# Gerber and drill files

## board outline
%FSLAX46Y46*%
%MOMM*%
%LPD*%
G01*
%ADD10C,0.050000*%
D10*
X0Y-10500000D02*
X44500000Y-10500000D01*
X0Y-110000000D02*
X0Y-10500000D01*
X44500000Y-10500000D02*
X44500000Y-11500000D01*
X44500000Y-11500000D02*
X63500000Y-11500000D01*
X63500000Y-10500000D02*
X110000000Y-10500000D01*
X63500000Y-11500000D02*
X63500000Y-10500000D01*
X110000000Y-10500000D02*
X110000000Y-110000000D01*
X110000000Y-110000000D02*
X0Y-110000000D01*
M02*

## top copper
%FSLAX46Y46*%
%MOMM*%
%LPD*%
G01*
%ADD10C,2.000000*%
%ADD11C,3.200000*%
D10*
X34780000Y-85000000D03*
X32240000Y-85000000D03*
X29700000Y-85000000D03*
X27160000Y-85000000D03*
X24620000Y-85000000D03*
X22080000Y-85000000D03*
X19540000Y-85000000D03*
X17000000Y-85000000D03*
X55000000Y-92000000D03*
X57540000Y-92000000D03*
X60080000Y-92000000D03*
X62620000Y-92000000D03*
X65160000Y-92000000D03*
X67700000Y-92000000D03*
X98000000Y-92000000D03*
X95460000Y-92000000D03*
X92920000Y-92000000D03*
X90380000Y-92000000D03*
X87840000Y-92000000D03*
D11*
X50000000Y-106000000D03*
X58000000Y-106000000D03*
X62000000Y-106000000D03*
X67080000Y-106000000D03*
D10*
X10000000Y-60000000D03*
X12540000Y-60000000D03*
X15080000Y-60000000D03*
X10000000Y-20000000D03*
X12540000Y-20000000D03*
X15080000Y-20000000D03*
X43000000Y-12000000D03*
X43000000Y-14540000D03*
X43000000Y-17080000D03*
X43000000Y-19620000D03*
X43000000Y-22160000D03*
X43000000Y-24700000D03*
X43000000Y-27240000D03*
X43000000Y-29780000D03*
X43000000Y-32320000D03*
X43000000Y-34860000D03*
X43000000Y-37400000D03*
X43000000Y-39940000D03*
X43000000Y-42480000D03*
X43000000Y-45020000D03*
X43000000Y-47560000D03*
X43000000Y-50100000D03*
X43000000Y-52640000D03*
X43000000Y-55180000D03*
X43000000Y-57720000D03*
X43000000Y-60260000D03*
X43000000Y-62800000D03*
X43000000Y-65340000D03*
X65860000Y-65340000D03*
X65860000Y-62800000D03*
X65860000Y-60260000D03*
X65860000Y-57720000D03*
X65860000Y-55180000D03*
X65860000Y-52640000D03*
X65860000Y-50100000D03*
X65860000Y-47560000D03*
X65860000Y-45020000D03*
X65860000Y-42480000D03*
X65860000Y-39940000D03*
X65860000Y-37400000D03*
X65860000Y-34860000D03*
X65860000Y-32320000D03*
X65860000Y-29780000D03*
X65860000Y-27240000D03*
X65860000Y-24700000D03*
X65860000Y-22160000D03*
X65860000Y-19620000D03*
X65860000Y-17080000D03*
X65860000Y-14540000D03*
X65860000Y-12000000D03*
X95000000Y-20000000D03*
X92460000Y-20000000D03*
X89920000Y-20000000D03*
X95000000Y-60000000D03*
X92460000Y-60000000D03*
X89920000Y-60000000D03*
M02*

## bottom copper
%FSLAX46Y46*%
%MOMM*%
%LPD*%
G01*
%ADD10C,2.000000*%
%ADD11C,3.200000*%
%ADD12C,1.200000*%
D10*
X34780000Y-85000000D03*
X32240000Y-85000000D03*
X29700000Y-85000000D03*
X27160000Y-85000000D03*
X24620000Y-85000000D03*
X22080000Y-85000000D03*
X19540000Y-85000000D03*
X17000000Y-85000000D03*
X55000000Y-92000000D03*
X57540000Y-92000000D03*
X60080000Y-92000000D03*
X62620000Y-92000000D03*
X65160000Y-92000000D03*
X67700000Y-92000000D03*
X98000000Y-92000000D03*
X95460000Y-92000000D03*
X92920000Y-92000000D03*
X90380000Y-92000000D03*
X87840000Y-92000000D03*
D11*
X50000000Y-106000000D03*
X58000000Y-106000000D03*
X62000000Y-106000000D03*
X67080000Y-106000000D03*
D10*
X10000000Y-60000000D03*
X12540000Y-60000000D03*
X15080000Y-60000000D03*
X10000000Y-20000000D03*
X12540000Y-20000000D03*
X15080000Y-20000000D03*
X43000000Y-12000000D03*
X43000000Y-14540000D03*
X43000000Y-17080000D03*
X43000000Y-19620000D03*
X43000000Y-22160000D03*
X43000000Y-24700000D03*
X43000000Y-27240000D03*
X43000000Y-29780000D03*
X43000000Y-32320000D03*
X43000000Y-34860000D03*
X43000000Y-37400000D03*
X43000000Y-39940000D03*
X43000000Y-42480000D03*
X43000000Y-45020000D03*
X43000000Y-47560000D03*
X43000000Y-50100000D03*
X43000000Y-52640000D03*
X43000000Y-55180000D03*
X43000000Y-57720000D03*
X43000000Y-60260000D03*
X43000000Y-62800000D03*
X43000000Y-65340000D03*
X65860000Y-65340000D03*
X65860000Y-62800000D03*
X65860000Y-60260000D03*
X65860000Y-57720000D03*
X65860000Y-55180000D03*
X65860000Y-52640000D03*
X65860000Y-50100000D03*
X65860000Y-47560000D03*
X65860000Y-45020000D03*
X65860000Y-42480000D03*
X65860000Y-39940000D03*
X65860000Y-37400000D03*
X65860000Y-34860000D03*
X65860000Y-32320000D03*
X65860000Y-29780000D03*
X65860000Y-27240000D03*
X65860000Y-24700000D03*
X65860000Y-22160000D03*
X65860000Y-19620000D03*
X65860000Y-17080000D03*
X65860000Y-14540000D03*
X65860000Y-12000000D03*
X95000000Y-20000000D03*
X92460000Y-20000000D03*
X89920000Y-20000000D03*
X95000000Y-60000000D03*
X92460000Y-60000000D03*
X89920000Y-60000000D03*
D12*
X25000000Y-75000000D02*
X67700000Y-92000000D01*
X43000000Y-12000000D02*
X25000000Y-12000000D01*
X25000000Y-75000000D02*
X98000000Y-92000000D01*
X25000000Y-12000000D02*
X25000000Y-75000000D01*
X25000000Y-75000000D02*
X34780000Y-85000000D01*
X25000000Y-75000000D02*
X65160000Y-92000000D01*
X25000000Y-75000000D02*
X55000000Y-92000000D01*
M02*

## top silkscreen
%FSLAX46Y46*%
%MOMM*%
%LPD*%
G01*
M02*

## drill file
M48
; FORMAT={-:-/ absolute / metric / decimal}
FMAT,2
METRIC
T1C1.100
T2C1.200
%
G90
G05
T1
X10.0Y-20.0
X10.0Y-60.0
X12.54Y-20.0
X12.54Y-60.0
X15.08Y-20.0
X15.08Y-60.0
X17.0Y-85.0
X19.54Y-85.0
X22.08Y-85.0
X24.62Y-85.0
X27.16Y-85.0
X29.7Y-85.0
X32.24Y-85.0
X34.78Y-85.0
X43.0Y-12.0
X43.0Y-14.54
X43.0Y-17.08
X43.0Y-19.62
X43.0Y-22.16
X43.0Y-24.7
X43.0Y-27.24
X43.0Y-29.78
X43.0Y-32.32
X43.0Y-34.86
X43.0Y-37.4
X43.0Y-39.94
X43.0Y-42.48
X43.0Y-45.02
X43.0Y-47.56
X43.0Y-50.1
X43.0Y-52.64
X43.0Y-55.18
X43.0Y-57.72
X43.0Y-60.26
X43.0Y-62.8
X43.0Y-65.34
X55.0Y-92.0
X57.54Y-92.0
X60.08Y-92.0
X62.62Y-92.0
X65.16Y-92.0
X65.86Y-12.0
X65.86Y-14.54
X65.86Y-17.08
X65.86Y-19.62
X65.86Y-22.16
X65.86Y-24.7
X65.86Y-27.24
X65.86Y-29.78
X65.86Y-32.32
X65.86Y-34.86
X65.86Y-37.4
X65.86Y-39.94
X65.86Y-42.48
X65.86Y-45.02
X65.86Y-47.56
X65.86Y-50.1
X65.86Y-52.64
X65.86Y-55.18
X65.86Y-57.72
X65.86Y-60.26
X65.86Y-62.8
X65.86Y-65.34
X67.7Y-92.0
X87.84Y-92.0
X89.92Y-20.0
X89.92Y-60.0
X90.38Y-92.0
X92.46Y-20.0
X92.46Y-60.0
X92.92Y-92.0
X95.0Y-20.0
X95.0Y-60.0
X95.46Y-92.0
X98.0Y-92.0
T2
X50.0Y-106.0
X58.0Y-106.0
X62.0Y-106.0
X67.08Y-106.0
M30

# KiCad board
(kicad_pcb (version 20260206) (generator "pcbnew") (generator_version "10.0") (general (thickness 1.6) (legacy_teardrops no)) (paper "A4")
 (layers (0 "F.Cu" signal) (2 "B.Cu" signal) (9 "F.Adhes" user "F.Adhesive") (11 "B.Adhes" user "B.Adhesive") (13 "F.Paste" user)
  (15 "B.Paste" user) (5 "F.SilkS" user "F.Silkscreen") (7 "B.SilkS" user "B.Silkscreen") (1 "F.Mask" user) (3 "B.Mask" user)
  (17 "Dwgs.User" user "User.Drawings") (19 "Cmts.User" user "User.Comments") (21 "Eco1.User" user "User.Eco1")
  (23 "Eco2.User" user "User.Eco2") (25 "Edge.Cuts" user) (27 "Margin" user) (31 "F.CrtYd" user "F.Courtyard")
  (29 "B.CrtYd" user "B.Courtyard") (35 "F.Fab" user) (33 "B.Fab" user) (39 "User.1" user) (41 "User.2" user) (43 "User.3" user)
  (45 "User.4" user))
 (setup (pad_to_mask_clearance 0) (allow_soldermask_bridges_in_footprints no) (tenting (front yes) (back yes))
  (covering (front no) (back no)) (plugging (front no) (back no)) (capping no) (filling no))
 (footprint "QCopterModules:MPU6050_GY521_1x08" (layer "F.Cu") (at 34.78 85 -90)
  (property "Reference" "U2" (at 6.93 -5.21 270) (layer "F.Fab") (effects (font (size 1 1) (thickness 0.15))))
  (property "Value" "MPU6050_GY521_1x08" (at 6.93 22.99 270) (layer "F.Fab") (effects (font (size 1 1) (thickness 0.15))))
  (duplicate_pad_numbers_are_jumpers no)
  (pad "1" thru_hole circle (at 0 0 270) (size 2 2) (drill 1.1) (layers "*.Cu" "*.Mask") (remove_unused_layers no) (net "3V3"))
  (pad "2" thru_hole circle (at 0 2.54 270) (size 2 2) (drill 1.1) (layers "*.Cu" "*.Mask") (remove_unused_layers no) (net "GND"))
  (pad "3" thru_hole circle (at 0 5.08 270) (size 2 2) (drill 1.1) (layers "*.Cu" "*.Mask") (remove_unused_layers no) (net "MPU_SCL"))
  (pad "4" thru_hole circle (at 0 7.62 270) (size 2 2) (drill 1.1) (layers "*.Cu" "*.Mask") (remove_unused_layers no) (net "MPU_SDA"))
  (pad "5" thru_hole circle (at 0 10.16 270) (size 2 2) (drill 1.1) (layers "*.Cu" "*.Mask") (remove_unused_layers no)
   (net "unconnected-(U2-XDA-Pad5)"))
  (pad "6" thru_hole circle (at 0 12.7 270) (size 2 2) (drill 1.1) (layers "*.Cu" "*.Mask") (remove_unused_layers no)
   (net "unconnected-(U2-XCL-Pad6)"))
  (pad "7" thru_hole circle (at 0 15.24 270) (size 2 2) (drill 1.1) (layers "*.Cu" "*.Mask") (remove_unused_layers no) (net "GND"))
  (pad "8" thru_hole circle (at 0 17.78 270) (size 2 2) (drill 1.1) (layers "*.Cu" "*.Mask") (remove_unused_layers no) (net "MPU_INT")))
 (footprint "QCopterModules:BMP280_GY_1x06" (layer "F.Cu") (at 55 92 90)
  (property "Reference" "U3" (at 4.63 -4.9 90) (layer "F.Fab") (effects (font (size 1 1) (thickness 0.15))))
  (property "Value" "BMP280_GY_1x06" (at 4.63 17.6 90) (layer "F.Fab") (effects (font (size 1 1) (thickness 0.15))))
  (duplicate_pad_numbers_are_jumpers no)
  (pad "1" thru_hole circle (at 0 0 90) (size 2 2) (drill 1.1) (layers "*.Cu" "*.Mask") (remove_unused_layers no) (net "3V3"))
  (pad "2" thru_hole circle (at 0 2.54 90) (size 2 2) (drill 1.1) (layers "*.Cu" "*.Mask") (remove_unused_layers no) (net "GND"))
  (pad "3" thru_hole circle (at 0 5.08 90) (size 2 2) (drill 1.1) (layers "*.Cu" "*.Mask") (remove_unused_layers no) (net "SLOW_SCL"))
  (pad "4" thru_hole circle (at 0 7.62 90) (size 2 2) (drill 1.1) (layers "*.Cu" "*.Mask") (remove_unused_layers no) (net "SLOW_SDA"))
  (pad "5" thru_hole circle (at 0 10.16 90) (size 2 2) (drill 1.1) (layers "*.Cu" "*.Mask") (remove_unused_layers no) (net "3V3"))
  (pad "6" thru_hole circle (at 0 12.7 90) (size 2 2) (drill 1.1) (layers "*.Cu" "*.Mask") (remove_unused_layers no) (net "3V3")))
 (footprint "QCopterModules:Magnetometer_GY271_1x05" (layer "F.Cu") (at 98 92 -90)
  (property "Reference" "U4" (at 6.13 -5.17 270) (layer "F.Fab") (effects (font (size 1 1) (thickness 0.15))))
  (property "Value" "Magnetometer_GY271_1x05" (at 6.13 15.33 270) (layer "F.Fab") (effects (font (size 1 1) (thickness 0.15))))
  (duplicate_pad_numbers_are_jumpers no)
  (pad "1" thru_hole circle (at 0 0 270) (size 2 2) (drill 1.1) (layers "*.Cu" "*.Mask") (remove_unused_layers no) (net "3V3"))
  (pad "2" thru_hole circle (at 0 2.54 270) (size 2 2) (drill 1.1) (layers "*.Cu" "*.Mask") (remove_unused_layers no) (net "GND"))
  (pad "3" thru_hole circle (at 0 5.08 270) (size 2 2) (drill 1.1) (layers "*.Cu" "*.Mask") (remove_unused_layers no) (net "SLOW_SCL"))
  (pad "4" thru_hole circle (at 0 7.62 270) (size 2 2) (drill 1.1) (layers "*.Cu" "*.Mask") (remove_unused_layers no) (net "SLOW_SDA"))
  (pad "5" thru_hole circle (at 0 10.16 270) (size 2 2) (drill 1.1) (layers "*.Cu" "*.Mask") (remove_unused_layers no) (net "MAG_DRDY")))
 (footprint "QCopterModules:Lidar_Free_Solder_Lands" (layer "F.Cu") (at 50 106)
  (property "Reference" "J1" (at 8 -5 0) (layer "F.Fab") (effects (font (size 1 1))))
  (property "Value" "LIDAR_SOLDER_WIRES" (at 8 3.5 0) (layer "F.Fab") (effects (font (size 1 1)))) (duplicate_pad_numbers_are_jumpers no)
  (pad "1" thru_hole circle (at 0 0) (size 3.2 3.2) (drill 1.2) (layers "*.Cu" "*.Mask") (remove_unused_layers no) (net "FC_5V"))
  (pad "2" thru_hole circle (at 8 0) (size 3.2 3.2) (drill 1.2) (layers "*.Cu" "*.Mask") (remove_unused_layers no) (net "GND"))
  (pad "3" thru_hole circle (at 12 0) (size 3.2 3.2) (drill 1.2) (layers "*.Cu" "*.Mask") (remove_unused_layers no) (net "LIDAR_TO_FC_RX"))
  (pad "4" thru_hole circle (at 17.08 0) (size 3.2 3.2) (drill 1.2) (layers "*.Cu" "*.Mask") (remove_unused_layers no)
   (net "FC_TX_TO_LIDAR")))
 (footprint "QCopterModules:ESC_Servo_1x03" (layer "F.Cu") (at 10 60 90)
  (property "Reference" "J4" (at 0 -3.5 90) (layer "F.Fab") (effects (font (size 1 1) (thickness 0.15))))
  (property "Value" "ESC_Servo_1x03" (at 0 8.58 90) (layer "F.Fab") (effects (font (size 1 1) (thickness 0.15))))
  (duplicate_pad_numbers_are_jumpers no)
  (pad "1" thru_hole circle (at 0 0 90) (size 2 2) (drill 1.1) (layers "*.Cu" "*.Mask") (remove_unused_layers no) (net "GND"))
  (pad "2" thru_hole circle (at 0 2.54 90) (size 2 2) (drill 1.1) (layers "*.Cu" "*.Mask") (remove_unused_layers no) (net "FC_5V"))
  (pad "3" thru_hole circle (at 0 5.08 90) (size 2 2) (drill 1.1) (layers "*.Cu" "*.Mask") (remove_unused_layers no) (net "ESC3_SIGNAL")))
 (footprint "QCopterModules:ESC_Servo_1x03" (layer "F.Cu") (at 10 20 90)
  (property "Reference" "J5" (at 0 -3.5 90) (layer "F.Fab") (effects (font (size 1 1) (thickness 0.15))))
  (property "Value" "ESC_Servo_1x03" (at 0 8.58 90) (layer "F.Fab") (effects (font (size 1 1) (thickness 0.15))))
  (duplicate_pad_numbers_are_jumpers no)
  (pad "1" thru_hole circle (at 0 0 90) (size 2 2) (drill 1.1) (layers "*.Cu" "*.Mask") (remove_unused_layers no) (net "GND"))
  (pad "2" thru_hole circle (at 0 2.54 90) (size 2 2) (drill 1.1) (layers "*.Cu" "*.Mask") (remove_unused_layers no)
   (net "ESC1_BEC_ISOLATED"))
  (pad "3" thru_hole circle (at 0 5.08 90) (size 2 2) (drill 1.1) (layers "*.Cu" "*.Mask") (remove_unused_layers no) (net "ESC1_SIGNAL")))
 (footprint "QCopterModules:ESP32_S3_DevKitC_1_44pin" (layer "F.Cu") (at 43 12)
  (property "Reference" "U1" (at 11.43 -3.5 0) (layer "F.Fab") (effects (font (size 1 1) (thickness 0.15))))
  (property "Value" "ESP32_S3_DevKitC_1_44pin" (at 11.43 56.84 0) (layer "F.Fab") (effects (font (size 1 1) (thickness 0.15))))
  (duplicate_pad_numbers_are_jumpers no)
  (pad "1" thru_hole circle (at 0 0) (size 2 2) (drill 1.1) (layers "*.Cu" "*.Mask") (remove_unused_layers no) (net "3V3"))
  (pad "2" thru_hole circle (at 0 2.54) (size 2 2) (drill 1.1) (layers "*.Cu" "*.Mask") (remove_unused_layers no))
  (pad "3" thru_hole circle (at 0 5.08) (size 2 2) (drill 1.1) (layers "*.Cu" "*.Mask") (remove_unused_layers no)
   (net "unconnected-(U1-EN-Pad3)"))
  (pad "4" thru_hole circle (at 0 7.62) (size 2 2) (drill 1.1) (layers "*.Cu" "*.Mask") (remove_unused_layers no) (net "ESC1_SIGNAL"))
  (pad "5" thru_hole circle (at 0 10.16) (size 2 2) (drill 1.1) (layers "*.Cu" "*.Mask") (remove_unused_layers no)
   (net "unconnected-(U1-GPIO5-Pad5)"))
  (pad "6" thru_hole circle (at 0 12.7) (size 2 2) (drill 1.1) (layers "*.Cu" "*.Mask") (remove_unused_layers no)
   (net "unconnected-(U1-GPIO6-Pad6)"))
  (pad "7" thru_hole circle (at 0 15.24) (size 2 2) (drill 1.1) (layers "*.Cu" "*.Mask") (remove_unused_layers no)
   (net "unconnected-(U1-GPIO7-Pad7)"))
  (pad "8" thru_hole circle (at 0 17.78) (size 2 2) (drill 1.1) (layers "*.Cu" "*.Mask") (remove_unused_layers no) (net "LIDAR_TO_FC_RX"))
  (pad "9" thru_hole circle (at 0 20.32) (size 2 2) (drill 1.1) (layers "*.Cu" "*.Mask") (remove_unused_layers no) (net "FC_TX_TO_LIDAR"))
  (pad "10" thru_hole circle (at 0 22.86) (size 2 2) (drill 1.1) (layers "*.Cu" "*.Mask") (remove_unused_layers no)
   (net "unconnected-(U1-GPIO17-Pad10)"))
  (pad "11" thru_hole circle (at 0 25.4) (size 2 2) (drill 1.1) (layers "*.Cu" "*.Mask") (remove_unused_layers no) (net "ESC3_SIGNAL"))
  (pad "12" thru_hole circle (at 0 27.94) (size 2 2) (drill 1.1) (layers "*.Cu" "*.Mask") (remove_unused_layers no)
   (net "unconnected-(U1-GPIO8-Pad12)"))
  (pad "13" thru_hole circle (at 0 30.48) (size 2 2) (drill 1.1) (layers "*.Cu" "*.Mask") (remove_unused_layers no)
   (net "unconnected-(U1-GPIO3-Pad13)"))
  (pad "14" thru_hole circle (at 0 33.02) (size 2 2) (drill 1.1) (layers "*.Cu" "*.Mask") (remove_unused_layers no)
   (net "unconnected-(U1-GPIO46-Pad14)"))
  (pad "15" thru_hole circle (at 0 35.56) (size 2 2) (drill 1.1) (layers "*.Cu" "*.Mask") (remove_unused_layers no)
   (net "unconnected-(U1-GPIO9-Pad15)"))
  (pad "16" thru_hole circle (at 0 38.1) (size 2 2) (drill 1.1) (layers "*.Cu" "*.Mask") (remove_unused_layers no)
   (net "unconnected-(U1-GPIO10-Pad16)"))
  (pad "17" thru_hole circle (at 0 40.64) (size 2 2) (drill 1.1) (layers "*.Cu" "*.Mask") (remove_unused_layers no)
   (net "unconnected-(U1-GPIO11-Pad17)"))
  (pad "18" thru_hole circle (at 0 43.18) (size 2 2) (drill 1.1) (layers "*.Cu" "*.Mask") (remove_unused_layers no) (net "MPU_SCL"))
  (pad "19" thru_hole circle (at 0 45.72) (size 2 2) (drill 1.1) (layers "*.Cu" "*.Mask") (remove_unused_layers no) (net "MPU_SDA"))
  (pad "20" thru_hole circle (at 0 48.26) (size 2 2) (drill 1.1) (layers "*.Cu" "*.Mask") (remove_unused_layers no) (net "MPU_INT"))
  (pad "21" thru_hole circle (at 0 50.8) (size 2 2) (drill 1.1) (layers "*.Cu" "*.Mask") (remove_unused_layers no) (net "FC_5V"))
  (pad "22" thru_hole circle (at 0 53.34) (size 2 2) (drill 1.1) (layers "*.Cu" "*.Mask") (remove_unused_layers no) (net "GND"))
  (pad "23" thru_hole circle (at 22.86 53.34) (size 2 2) (drill 1.1) (layers "*.Cu" "*.Mask") (remove_unused_layers no) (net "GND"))
  (pad "24" thru_hole circle (at 22.86 50.8) (size 2 2) (drill 1.1) (layers "*.Cu" "*.Mask") (remove_unused_layers no) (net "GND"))
  (pad "25" thru_hole circle (at 22.86 48.26) (size 2 2) (drill 1.1) (layers "*.Cu" "*.Mask") (remove_unused_layers no)
   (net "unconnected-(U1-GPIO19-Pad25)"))
  (pad "26" thru_hole circle (at 22.86 45.72) (size 2 2) (drill 1.1) (layers "*.Cu" "*.Mask") (remove_unused_layers no)
   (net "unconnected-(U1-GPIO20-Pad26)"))
  (pad "27" thru_hole circle (at 22.86 43.18) (size 2 2) (drill 1.1) (layers "*.Cu" "*.Mask") (remove_unused_layers no) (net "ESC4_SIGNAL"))
  (pad "28" thru_hole circle (at 22.86 40.64) (size 2 2) (drill 1.1) (layers "*.Cu" "*.Mask") (remove_unused_layers no)
   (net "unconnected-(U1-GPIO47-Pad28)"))
  (pad "29" thru_hole circle (at 22.86 38.1) (size 2 2) (drill 1.1) (layers "*.Cu" "*.Mask") (remove_unused_layers no)
   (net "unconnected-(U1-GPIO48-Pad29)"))
  (pad "30" thru_hole circle (at 22.86 35.56) (size 2 2) (drill 1.1) (layers "*.Cu" "*.Mask") (remove_unused_layers no)
   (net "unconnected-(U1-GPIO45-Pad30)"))
  (pad "31" thru_hole circle (at 22.86 33.02) (size 2 2) (drill 1.1) (layers "*.Cu" "*.Mask") (remove_unused_layers no)
   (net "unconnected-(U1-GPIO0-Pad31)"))
  (pad "32" thru_hole circle (at 22.86 30.48) (size 2 2) (drill 1.1) (layers "*.Cu" "*.Mask") (remove_unused_layers no)
   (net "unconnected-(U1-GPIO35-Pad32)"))
  (pad "33" thru_hole circle (at 22.86 27.94) (size 2 2) (drill 1.1) (layers "*.Cu" "*.Mask") (remove_unused_layers no)
   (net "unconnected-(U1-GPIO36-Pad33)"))
  (pad "34" thru_hole circle (at 22.86 25.4) (size 2 2) (drill 1.1) (layers "*.Cu" "*.Mask") (remove_unused_layers no)
   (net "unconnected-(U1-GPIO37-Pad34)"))
  (pad "35" thru_hole circle (at 22.86 22.86) (size 2 2) (drill 1.1) (layers "*.Cu" "*.Mask") (remove_unused_layers no)
   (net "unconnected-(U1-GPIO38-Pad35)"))
  (pad "36" thru_hole circle (at 22.86 20.32) (size 2 2) (drill 1.1) (layers "*.Cu" "*.Mask") (remove_unused_layers no) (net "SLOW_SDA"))
  (pad "37" thru_hole circle (at 22.86 17.78) (size 2 2) (drill 1.1) (layers "*.Cu" "*.Mask") (remove_unused_layers no) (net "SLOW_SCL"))
  (pad "38" thru_hole circle (at 22.86 15.24) (size 2 2) (drill 1.1) (layers "*.Cu" "*.Mask") (remove_unused_layers no) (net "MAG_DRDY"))
  (pad "39" thru_hole circle (at 22.86 12.7) (size 2 2) (drill 1.1) (layers "*.Cu" "*.Mask") (remove_unused_layers no)
   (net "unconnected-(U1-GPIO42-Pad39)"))
  (pad "40" thru_hole circle (at 22.86 10.16) (size 2 2) (drill 1.1) (layers "*.Cu" "*.Mask") (remove_unused_layers no) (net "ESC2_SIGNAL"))
  (pad "41" thru_hole circle (at 22.86 7.62) (size 2 2) (drill 1.1) (layers "*.Cu" "*.Mask") (remove_unused_layers no)
   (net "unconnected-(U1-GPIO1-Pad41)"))
  (pad "42" thru_hole circle (at 22.86 5.08) (size 2 2) (drill 1.1) (layers "*.Cu" "*.Mask") (remove_unused_layers no)
   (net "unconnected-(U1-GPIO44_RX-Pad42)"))
  (pad "43" thru_hole circle (at 22.86 2.54) (size 2 2) (drill 1.1) (layers "*.Cu" "*.Mask") (remove_unused_layers no)
   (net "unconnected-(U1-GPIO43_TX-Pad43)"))
  (pad "44" thru_hole circle (at 22.86 0) (size 2 2) (drill 1.1) (layers "*.Cu" "*.Mask") (remove_unused_layers no) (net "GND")))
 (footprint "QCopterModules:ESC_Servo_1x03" (layer "F.Cu") (at 95 20 -90)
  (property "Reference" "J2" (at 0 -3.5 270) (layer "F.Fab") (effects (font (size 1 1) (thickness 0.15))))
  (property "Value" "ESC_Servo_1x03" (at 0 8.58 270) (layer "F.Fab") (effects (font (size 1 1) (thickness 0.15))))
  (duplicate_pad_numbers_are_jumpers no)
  (pad "1" thru_hole circle (at 0 0 270) (size 2 2) (drill 1.1) (layers "*.Cu" "*.Mask") (remove_unused_layers no) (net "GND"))
  (pad "2" thru_hole circle (at 0 2.54 270) (size 2 2) (drill 1.1) (layers "*.Cu" "*.Mask") (remove_unused_layers no)
   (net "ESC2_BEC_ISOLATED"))
  (pad "3" thru_hole circle (at 0 5.08 270) (size 2 2) (drill 1.1) (layers "*.Cu" "*.Mask") (remove_unused_layers no) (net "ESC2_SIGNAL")))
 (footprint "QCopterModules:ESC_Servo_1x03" (layer "F.Cu") (at 95 60 -90)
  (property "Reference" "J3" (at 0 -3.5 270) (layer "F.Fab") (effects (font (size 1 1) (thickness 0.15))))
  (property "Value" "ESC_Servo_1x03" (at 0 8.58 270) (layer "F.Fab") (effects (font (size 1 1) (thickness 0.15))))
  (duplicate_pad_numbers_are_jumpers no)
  (pad "1" thru_hole circle (at 0 0 270) (size 2 2) (drill 1.1) (layers "*.Cu" "*.Mask") (remove_unused_layers no) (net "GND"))
  (pad "2" thru_hole circle (at 0 2.54 270) (size 2 2) (drill 1.1) (layers "*.Cu" "*.Mask") (remove_unused_layers no)
   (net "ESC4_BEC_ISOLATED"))
  (pad "3" thru_hole circle (at 0 5.08 270) (size 2 2) (drill 1.1) (layers "*.Cu" "*.Mask") (remove_unused_layers no) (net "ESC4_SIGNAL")))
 (gr_line (start 0 10.5) (end 44.5 10.5) (stroke (width 0.05) (type default)) (layer "Edge.Cuts"))
 (gr_line (start 0 110) (end 0 10.5) (stroke (width 0.05) (type default)) (layer "Edge.Cuts"))
 (gr_line (start 44.5 10.5) (end 44.5 11.5) (stroke (width 0.05) (type default)) (layer "Edge.Cuts"))
 (gr_line (start 44.5 11.5) (end 63.5 11.5) (stroke (width 0.05) (type default)) (layer "Edge.Cuts"))
 (gr_line (start 63.5 10.5) (end 110 10.5) (stroke (width 0.05) (type default)) (layer "Edge.Cuts"))
 (gr_line (start 63.5 11.5) (end 63.5 10.5) (stroke (width 0.05) (type default)) (layer "Edge.Cuts"))
 (gr_line (start 110 10.5) (end 110 110) (stroke (width 0.05) (type default)) (layer "Edge.Cuts"))
 (gr_line (start 110 110) (end 0 110) (stroke (width 0.05) (type default)) (layer "Edge.Cuts"))
 (segment (start 25 75) (end 67.7 92) (width 1.2) (layer "B.Cu") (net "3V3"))
 (segment (start 43 12) (end 25 12) (width 1.2) (layer "B.Cu") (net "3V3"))
 (segment (start 25 75) (end 98 92) (width 1.2) (layer "B.Cu") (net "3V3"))
 (segment (start 25 12) (end 25 75) (width 1.2) (layer "B.Cu") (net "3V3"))
 (segment (start 25 75) (end 34.78 85) (width 1.2) (layer "B.Cu") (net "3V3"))
 (segment (start 25 75) (end 65.16 92) (width 1.2) (layer "B.Cu") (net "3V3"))
 (segment (start 25 75) (end 55 92) (width 1.2) (layer "B.Cu") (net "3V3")))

